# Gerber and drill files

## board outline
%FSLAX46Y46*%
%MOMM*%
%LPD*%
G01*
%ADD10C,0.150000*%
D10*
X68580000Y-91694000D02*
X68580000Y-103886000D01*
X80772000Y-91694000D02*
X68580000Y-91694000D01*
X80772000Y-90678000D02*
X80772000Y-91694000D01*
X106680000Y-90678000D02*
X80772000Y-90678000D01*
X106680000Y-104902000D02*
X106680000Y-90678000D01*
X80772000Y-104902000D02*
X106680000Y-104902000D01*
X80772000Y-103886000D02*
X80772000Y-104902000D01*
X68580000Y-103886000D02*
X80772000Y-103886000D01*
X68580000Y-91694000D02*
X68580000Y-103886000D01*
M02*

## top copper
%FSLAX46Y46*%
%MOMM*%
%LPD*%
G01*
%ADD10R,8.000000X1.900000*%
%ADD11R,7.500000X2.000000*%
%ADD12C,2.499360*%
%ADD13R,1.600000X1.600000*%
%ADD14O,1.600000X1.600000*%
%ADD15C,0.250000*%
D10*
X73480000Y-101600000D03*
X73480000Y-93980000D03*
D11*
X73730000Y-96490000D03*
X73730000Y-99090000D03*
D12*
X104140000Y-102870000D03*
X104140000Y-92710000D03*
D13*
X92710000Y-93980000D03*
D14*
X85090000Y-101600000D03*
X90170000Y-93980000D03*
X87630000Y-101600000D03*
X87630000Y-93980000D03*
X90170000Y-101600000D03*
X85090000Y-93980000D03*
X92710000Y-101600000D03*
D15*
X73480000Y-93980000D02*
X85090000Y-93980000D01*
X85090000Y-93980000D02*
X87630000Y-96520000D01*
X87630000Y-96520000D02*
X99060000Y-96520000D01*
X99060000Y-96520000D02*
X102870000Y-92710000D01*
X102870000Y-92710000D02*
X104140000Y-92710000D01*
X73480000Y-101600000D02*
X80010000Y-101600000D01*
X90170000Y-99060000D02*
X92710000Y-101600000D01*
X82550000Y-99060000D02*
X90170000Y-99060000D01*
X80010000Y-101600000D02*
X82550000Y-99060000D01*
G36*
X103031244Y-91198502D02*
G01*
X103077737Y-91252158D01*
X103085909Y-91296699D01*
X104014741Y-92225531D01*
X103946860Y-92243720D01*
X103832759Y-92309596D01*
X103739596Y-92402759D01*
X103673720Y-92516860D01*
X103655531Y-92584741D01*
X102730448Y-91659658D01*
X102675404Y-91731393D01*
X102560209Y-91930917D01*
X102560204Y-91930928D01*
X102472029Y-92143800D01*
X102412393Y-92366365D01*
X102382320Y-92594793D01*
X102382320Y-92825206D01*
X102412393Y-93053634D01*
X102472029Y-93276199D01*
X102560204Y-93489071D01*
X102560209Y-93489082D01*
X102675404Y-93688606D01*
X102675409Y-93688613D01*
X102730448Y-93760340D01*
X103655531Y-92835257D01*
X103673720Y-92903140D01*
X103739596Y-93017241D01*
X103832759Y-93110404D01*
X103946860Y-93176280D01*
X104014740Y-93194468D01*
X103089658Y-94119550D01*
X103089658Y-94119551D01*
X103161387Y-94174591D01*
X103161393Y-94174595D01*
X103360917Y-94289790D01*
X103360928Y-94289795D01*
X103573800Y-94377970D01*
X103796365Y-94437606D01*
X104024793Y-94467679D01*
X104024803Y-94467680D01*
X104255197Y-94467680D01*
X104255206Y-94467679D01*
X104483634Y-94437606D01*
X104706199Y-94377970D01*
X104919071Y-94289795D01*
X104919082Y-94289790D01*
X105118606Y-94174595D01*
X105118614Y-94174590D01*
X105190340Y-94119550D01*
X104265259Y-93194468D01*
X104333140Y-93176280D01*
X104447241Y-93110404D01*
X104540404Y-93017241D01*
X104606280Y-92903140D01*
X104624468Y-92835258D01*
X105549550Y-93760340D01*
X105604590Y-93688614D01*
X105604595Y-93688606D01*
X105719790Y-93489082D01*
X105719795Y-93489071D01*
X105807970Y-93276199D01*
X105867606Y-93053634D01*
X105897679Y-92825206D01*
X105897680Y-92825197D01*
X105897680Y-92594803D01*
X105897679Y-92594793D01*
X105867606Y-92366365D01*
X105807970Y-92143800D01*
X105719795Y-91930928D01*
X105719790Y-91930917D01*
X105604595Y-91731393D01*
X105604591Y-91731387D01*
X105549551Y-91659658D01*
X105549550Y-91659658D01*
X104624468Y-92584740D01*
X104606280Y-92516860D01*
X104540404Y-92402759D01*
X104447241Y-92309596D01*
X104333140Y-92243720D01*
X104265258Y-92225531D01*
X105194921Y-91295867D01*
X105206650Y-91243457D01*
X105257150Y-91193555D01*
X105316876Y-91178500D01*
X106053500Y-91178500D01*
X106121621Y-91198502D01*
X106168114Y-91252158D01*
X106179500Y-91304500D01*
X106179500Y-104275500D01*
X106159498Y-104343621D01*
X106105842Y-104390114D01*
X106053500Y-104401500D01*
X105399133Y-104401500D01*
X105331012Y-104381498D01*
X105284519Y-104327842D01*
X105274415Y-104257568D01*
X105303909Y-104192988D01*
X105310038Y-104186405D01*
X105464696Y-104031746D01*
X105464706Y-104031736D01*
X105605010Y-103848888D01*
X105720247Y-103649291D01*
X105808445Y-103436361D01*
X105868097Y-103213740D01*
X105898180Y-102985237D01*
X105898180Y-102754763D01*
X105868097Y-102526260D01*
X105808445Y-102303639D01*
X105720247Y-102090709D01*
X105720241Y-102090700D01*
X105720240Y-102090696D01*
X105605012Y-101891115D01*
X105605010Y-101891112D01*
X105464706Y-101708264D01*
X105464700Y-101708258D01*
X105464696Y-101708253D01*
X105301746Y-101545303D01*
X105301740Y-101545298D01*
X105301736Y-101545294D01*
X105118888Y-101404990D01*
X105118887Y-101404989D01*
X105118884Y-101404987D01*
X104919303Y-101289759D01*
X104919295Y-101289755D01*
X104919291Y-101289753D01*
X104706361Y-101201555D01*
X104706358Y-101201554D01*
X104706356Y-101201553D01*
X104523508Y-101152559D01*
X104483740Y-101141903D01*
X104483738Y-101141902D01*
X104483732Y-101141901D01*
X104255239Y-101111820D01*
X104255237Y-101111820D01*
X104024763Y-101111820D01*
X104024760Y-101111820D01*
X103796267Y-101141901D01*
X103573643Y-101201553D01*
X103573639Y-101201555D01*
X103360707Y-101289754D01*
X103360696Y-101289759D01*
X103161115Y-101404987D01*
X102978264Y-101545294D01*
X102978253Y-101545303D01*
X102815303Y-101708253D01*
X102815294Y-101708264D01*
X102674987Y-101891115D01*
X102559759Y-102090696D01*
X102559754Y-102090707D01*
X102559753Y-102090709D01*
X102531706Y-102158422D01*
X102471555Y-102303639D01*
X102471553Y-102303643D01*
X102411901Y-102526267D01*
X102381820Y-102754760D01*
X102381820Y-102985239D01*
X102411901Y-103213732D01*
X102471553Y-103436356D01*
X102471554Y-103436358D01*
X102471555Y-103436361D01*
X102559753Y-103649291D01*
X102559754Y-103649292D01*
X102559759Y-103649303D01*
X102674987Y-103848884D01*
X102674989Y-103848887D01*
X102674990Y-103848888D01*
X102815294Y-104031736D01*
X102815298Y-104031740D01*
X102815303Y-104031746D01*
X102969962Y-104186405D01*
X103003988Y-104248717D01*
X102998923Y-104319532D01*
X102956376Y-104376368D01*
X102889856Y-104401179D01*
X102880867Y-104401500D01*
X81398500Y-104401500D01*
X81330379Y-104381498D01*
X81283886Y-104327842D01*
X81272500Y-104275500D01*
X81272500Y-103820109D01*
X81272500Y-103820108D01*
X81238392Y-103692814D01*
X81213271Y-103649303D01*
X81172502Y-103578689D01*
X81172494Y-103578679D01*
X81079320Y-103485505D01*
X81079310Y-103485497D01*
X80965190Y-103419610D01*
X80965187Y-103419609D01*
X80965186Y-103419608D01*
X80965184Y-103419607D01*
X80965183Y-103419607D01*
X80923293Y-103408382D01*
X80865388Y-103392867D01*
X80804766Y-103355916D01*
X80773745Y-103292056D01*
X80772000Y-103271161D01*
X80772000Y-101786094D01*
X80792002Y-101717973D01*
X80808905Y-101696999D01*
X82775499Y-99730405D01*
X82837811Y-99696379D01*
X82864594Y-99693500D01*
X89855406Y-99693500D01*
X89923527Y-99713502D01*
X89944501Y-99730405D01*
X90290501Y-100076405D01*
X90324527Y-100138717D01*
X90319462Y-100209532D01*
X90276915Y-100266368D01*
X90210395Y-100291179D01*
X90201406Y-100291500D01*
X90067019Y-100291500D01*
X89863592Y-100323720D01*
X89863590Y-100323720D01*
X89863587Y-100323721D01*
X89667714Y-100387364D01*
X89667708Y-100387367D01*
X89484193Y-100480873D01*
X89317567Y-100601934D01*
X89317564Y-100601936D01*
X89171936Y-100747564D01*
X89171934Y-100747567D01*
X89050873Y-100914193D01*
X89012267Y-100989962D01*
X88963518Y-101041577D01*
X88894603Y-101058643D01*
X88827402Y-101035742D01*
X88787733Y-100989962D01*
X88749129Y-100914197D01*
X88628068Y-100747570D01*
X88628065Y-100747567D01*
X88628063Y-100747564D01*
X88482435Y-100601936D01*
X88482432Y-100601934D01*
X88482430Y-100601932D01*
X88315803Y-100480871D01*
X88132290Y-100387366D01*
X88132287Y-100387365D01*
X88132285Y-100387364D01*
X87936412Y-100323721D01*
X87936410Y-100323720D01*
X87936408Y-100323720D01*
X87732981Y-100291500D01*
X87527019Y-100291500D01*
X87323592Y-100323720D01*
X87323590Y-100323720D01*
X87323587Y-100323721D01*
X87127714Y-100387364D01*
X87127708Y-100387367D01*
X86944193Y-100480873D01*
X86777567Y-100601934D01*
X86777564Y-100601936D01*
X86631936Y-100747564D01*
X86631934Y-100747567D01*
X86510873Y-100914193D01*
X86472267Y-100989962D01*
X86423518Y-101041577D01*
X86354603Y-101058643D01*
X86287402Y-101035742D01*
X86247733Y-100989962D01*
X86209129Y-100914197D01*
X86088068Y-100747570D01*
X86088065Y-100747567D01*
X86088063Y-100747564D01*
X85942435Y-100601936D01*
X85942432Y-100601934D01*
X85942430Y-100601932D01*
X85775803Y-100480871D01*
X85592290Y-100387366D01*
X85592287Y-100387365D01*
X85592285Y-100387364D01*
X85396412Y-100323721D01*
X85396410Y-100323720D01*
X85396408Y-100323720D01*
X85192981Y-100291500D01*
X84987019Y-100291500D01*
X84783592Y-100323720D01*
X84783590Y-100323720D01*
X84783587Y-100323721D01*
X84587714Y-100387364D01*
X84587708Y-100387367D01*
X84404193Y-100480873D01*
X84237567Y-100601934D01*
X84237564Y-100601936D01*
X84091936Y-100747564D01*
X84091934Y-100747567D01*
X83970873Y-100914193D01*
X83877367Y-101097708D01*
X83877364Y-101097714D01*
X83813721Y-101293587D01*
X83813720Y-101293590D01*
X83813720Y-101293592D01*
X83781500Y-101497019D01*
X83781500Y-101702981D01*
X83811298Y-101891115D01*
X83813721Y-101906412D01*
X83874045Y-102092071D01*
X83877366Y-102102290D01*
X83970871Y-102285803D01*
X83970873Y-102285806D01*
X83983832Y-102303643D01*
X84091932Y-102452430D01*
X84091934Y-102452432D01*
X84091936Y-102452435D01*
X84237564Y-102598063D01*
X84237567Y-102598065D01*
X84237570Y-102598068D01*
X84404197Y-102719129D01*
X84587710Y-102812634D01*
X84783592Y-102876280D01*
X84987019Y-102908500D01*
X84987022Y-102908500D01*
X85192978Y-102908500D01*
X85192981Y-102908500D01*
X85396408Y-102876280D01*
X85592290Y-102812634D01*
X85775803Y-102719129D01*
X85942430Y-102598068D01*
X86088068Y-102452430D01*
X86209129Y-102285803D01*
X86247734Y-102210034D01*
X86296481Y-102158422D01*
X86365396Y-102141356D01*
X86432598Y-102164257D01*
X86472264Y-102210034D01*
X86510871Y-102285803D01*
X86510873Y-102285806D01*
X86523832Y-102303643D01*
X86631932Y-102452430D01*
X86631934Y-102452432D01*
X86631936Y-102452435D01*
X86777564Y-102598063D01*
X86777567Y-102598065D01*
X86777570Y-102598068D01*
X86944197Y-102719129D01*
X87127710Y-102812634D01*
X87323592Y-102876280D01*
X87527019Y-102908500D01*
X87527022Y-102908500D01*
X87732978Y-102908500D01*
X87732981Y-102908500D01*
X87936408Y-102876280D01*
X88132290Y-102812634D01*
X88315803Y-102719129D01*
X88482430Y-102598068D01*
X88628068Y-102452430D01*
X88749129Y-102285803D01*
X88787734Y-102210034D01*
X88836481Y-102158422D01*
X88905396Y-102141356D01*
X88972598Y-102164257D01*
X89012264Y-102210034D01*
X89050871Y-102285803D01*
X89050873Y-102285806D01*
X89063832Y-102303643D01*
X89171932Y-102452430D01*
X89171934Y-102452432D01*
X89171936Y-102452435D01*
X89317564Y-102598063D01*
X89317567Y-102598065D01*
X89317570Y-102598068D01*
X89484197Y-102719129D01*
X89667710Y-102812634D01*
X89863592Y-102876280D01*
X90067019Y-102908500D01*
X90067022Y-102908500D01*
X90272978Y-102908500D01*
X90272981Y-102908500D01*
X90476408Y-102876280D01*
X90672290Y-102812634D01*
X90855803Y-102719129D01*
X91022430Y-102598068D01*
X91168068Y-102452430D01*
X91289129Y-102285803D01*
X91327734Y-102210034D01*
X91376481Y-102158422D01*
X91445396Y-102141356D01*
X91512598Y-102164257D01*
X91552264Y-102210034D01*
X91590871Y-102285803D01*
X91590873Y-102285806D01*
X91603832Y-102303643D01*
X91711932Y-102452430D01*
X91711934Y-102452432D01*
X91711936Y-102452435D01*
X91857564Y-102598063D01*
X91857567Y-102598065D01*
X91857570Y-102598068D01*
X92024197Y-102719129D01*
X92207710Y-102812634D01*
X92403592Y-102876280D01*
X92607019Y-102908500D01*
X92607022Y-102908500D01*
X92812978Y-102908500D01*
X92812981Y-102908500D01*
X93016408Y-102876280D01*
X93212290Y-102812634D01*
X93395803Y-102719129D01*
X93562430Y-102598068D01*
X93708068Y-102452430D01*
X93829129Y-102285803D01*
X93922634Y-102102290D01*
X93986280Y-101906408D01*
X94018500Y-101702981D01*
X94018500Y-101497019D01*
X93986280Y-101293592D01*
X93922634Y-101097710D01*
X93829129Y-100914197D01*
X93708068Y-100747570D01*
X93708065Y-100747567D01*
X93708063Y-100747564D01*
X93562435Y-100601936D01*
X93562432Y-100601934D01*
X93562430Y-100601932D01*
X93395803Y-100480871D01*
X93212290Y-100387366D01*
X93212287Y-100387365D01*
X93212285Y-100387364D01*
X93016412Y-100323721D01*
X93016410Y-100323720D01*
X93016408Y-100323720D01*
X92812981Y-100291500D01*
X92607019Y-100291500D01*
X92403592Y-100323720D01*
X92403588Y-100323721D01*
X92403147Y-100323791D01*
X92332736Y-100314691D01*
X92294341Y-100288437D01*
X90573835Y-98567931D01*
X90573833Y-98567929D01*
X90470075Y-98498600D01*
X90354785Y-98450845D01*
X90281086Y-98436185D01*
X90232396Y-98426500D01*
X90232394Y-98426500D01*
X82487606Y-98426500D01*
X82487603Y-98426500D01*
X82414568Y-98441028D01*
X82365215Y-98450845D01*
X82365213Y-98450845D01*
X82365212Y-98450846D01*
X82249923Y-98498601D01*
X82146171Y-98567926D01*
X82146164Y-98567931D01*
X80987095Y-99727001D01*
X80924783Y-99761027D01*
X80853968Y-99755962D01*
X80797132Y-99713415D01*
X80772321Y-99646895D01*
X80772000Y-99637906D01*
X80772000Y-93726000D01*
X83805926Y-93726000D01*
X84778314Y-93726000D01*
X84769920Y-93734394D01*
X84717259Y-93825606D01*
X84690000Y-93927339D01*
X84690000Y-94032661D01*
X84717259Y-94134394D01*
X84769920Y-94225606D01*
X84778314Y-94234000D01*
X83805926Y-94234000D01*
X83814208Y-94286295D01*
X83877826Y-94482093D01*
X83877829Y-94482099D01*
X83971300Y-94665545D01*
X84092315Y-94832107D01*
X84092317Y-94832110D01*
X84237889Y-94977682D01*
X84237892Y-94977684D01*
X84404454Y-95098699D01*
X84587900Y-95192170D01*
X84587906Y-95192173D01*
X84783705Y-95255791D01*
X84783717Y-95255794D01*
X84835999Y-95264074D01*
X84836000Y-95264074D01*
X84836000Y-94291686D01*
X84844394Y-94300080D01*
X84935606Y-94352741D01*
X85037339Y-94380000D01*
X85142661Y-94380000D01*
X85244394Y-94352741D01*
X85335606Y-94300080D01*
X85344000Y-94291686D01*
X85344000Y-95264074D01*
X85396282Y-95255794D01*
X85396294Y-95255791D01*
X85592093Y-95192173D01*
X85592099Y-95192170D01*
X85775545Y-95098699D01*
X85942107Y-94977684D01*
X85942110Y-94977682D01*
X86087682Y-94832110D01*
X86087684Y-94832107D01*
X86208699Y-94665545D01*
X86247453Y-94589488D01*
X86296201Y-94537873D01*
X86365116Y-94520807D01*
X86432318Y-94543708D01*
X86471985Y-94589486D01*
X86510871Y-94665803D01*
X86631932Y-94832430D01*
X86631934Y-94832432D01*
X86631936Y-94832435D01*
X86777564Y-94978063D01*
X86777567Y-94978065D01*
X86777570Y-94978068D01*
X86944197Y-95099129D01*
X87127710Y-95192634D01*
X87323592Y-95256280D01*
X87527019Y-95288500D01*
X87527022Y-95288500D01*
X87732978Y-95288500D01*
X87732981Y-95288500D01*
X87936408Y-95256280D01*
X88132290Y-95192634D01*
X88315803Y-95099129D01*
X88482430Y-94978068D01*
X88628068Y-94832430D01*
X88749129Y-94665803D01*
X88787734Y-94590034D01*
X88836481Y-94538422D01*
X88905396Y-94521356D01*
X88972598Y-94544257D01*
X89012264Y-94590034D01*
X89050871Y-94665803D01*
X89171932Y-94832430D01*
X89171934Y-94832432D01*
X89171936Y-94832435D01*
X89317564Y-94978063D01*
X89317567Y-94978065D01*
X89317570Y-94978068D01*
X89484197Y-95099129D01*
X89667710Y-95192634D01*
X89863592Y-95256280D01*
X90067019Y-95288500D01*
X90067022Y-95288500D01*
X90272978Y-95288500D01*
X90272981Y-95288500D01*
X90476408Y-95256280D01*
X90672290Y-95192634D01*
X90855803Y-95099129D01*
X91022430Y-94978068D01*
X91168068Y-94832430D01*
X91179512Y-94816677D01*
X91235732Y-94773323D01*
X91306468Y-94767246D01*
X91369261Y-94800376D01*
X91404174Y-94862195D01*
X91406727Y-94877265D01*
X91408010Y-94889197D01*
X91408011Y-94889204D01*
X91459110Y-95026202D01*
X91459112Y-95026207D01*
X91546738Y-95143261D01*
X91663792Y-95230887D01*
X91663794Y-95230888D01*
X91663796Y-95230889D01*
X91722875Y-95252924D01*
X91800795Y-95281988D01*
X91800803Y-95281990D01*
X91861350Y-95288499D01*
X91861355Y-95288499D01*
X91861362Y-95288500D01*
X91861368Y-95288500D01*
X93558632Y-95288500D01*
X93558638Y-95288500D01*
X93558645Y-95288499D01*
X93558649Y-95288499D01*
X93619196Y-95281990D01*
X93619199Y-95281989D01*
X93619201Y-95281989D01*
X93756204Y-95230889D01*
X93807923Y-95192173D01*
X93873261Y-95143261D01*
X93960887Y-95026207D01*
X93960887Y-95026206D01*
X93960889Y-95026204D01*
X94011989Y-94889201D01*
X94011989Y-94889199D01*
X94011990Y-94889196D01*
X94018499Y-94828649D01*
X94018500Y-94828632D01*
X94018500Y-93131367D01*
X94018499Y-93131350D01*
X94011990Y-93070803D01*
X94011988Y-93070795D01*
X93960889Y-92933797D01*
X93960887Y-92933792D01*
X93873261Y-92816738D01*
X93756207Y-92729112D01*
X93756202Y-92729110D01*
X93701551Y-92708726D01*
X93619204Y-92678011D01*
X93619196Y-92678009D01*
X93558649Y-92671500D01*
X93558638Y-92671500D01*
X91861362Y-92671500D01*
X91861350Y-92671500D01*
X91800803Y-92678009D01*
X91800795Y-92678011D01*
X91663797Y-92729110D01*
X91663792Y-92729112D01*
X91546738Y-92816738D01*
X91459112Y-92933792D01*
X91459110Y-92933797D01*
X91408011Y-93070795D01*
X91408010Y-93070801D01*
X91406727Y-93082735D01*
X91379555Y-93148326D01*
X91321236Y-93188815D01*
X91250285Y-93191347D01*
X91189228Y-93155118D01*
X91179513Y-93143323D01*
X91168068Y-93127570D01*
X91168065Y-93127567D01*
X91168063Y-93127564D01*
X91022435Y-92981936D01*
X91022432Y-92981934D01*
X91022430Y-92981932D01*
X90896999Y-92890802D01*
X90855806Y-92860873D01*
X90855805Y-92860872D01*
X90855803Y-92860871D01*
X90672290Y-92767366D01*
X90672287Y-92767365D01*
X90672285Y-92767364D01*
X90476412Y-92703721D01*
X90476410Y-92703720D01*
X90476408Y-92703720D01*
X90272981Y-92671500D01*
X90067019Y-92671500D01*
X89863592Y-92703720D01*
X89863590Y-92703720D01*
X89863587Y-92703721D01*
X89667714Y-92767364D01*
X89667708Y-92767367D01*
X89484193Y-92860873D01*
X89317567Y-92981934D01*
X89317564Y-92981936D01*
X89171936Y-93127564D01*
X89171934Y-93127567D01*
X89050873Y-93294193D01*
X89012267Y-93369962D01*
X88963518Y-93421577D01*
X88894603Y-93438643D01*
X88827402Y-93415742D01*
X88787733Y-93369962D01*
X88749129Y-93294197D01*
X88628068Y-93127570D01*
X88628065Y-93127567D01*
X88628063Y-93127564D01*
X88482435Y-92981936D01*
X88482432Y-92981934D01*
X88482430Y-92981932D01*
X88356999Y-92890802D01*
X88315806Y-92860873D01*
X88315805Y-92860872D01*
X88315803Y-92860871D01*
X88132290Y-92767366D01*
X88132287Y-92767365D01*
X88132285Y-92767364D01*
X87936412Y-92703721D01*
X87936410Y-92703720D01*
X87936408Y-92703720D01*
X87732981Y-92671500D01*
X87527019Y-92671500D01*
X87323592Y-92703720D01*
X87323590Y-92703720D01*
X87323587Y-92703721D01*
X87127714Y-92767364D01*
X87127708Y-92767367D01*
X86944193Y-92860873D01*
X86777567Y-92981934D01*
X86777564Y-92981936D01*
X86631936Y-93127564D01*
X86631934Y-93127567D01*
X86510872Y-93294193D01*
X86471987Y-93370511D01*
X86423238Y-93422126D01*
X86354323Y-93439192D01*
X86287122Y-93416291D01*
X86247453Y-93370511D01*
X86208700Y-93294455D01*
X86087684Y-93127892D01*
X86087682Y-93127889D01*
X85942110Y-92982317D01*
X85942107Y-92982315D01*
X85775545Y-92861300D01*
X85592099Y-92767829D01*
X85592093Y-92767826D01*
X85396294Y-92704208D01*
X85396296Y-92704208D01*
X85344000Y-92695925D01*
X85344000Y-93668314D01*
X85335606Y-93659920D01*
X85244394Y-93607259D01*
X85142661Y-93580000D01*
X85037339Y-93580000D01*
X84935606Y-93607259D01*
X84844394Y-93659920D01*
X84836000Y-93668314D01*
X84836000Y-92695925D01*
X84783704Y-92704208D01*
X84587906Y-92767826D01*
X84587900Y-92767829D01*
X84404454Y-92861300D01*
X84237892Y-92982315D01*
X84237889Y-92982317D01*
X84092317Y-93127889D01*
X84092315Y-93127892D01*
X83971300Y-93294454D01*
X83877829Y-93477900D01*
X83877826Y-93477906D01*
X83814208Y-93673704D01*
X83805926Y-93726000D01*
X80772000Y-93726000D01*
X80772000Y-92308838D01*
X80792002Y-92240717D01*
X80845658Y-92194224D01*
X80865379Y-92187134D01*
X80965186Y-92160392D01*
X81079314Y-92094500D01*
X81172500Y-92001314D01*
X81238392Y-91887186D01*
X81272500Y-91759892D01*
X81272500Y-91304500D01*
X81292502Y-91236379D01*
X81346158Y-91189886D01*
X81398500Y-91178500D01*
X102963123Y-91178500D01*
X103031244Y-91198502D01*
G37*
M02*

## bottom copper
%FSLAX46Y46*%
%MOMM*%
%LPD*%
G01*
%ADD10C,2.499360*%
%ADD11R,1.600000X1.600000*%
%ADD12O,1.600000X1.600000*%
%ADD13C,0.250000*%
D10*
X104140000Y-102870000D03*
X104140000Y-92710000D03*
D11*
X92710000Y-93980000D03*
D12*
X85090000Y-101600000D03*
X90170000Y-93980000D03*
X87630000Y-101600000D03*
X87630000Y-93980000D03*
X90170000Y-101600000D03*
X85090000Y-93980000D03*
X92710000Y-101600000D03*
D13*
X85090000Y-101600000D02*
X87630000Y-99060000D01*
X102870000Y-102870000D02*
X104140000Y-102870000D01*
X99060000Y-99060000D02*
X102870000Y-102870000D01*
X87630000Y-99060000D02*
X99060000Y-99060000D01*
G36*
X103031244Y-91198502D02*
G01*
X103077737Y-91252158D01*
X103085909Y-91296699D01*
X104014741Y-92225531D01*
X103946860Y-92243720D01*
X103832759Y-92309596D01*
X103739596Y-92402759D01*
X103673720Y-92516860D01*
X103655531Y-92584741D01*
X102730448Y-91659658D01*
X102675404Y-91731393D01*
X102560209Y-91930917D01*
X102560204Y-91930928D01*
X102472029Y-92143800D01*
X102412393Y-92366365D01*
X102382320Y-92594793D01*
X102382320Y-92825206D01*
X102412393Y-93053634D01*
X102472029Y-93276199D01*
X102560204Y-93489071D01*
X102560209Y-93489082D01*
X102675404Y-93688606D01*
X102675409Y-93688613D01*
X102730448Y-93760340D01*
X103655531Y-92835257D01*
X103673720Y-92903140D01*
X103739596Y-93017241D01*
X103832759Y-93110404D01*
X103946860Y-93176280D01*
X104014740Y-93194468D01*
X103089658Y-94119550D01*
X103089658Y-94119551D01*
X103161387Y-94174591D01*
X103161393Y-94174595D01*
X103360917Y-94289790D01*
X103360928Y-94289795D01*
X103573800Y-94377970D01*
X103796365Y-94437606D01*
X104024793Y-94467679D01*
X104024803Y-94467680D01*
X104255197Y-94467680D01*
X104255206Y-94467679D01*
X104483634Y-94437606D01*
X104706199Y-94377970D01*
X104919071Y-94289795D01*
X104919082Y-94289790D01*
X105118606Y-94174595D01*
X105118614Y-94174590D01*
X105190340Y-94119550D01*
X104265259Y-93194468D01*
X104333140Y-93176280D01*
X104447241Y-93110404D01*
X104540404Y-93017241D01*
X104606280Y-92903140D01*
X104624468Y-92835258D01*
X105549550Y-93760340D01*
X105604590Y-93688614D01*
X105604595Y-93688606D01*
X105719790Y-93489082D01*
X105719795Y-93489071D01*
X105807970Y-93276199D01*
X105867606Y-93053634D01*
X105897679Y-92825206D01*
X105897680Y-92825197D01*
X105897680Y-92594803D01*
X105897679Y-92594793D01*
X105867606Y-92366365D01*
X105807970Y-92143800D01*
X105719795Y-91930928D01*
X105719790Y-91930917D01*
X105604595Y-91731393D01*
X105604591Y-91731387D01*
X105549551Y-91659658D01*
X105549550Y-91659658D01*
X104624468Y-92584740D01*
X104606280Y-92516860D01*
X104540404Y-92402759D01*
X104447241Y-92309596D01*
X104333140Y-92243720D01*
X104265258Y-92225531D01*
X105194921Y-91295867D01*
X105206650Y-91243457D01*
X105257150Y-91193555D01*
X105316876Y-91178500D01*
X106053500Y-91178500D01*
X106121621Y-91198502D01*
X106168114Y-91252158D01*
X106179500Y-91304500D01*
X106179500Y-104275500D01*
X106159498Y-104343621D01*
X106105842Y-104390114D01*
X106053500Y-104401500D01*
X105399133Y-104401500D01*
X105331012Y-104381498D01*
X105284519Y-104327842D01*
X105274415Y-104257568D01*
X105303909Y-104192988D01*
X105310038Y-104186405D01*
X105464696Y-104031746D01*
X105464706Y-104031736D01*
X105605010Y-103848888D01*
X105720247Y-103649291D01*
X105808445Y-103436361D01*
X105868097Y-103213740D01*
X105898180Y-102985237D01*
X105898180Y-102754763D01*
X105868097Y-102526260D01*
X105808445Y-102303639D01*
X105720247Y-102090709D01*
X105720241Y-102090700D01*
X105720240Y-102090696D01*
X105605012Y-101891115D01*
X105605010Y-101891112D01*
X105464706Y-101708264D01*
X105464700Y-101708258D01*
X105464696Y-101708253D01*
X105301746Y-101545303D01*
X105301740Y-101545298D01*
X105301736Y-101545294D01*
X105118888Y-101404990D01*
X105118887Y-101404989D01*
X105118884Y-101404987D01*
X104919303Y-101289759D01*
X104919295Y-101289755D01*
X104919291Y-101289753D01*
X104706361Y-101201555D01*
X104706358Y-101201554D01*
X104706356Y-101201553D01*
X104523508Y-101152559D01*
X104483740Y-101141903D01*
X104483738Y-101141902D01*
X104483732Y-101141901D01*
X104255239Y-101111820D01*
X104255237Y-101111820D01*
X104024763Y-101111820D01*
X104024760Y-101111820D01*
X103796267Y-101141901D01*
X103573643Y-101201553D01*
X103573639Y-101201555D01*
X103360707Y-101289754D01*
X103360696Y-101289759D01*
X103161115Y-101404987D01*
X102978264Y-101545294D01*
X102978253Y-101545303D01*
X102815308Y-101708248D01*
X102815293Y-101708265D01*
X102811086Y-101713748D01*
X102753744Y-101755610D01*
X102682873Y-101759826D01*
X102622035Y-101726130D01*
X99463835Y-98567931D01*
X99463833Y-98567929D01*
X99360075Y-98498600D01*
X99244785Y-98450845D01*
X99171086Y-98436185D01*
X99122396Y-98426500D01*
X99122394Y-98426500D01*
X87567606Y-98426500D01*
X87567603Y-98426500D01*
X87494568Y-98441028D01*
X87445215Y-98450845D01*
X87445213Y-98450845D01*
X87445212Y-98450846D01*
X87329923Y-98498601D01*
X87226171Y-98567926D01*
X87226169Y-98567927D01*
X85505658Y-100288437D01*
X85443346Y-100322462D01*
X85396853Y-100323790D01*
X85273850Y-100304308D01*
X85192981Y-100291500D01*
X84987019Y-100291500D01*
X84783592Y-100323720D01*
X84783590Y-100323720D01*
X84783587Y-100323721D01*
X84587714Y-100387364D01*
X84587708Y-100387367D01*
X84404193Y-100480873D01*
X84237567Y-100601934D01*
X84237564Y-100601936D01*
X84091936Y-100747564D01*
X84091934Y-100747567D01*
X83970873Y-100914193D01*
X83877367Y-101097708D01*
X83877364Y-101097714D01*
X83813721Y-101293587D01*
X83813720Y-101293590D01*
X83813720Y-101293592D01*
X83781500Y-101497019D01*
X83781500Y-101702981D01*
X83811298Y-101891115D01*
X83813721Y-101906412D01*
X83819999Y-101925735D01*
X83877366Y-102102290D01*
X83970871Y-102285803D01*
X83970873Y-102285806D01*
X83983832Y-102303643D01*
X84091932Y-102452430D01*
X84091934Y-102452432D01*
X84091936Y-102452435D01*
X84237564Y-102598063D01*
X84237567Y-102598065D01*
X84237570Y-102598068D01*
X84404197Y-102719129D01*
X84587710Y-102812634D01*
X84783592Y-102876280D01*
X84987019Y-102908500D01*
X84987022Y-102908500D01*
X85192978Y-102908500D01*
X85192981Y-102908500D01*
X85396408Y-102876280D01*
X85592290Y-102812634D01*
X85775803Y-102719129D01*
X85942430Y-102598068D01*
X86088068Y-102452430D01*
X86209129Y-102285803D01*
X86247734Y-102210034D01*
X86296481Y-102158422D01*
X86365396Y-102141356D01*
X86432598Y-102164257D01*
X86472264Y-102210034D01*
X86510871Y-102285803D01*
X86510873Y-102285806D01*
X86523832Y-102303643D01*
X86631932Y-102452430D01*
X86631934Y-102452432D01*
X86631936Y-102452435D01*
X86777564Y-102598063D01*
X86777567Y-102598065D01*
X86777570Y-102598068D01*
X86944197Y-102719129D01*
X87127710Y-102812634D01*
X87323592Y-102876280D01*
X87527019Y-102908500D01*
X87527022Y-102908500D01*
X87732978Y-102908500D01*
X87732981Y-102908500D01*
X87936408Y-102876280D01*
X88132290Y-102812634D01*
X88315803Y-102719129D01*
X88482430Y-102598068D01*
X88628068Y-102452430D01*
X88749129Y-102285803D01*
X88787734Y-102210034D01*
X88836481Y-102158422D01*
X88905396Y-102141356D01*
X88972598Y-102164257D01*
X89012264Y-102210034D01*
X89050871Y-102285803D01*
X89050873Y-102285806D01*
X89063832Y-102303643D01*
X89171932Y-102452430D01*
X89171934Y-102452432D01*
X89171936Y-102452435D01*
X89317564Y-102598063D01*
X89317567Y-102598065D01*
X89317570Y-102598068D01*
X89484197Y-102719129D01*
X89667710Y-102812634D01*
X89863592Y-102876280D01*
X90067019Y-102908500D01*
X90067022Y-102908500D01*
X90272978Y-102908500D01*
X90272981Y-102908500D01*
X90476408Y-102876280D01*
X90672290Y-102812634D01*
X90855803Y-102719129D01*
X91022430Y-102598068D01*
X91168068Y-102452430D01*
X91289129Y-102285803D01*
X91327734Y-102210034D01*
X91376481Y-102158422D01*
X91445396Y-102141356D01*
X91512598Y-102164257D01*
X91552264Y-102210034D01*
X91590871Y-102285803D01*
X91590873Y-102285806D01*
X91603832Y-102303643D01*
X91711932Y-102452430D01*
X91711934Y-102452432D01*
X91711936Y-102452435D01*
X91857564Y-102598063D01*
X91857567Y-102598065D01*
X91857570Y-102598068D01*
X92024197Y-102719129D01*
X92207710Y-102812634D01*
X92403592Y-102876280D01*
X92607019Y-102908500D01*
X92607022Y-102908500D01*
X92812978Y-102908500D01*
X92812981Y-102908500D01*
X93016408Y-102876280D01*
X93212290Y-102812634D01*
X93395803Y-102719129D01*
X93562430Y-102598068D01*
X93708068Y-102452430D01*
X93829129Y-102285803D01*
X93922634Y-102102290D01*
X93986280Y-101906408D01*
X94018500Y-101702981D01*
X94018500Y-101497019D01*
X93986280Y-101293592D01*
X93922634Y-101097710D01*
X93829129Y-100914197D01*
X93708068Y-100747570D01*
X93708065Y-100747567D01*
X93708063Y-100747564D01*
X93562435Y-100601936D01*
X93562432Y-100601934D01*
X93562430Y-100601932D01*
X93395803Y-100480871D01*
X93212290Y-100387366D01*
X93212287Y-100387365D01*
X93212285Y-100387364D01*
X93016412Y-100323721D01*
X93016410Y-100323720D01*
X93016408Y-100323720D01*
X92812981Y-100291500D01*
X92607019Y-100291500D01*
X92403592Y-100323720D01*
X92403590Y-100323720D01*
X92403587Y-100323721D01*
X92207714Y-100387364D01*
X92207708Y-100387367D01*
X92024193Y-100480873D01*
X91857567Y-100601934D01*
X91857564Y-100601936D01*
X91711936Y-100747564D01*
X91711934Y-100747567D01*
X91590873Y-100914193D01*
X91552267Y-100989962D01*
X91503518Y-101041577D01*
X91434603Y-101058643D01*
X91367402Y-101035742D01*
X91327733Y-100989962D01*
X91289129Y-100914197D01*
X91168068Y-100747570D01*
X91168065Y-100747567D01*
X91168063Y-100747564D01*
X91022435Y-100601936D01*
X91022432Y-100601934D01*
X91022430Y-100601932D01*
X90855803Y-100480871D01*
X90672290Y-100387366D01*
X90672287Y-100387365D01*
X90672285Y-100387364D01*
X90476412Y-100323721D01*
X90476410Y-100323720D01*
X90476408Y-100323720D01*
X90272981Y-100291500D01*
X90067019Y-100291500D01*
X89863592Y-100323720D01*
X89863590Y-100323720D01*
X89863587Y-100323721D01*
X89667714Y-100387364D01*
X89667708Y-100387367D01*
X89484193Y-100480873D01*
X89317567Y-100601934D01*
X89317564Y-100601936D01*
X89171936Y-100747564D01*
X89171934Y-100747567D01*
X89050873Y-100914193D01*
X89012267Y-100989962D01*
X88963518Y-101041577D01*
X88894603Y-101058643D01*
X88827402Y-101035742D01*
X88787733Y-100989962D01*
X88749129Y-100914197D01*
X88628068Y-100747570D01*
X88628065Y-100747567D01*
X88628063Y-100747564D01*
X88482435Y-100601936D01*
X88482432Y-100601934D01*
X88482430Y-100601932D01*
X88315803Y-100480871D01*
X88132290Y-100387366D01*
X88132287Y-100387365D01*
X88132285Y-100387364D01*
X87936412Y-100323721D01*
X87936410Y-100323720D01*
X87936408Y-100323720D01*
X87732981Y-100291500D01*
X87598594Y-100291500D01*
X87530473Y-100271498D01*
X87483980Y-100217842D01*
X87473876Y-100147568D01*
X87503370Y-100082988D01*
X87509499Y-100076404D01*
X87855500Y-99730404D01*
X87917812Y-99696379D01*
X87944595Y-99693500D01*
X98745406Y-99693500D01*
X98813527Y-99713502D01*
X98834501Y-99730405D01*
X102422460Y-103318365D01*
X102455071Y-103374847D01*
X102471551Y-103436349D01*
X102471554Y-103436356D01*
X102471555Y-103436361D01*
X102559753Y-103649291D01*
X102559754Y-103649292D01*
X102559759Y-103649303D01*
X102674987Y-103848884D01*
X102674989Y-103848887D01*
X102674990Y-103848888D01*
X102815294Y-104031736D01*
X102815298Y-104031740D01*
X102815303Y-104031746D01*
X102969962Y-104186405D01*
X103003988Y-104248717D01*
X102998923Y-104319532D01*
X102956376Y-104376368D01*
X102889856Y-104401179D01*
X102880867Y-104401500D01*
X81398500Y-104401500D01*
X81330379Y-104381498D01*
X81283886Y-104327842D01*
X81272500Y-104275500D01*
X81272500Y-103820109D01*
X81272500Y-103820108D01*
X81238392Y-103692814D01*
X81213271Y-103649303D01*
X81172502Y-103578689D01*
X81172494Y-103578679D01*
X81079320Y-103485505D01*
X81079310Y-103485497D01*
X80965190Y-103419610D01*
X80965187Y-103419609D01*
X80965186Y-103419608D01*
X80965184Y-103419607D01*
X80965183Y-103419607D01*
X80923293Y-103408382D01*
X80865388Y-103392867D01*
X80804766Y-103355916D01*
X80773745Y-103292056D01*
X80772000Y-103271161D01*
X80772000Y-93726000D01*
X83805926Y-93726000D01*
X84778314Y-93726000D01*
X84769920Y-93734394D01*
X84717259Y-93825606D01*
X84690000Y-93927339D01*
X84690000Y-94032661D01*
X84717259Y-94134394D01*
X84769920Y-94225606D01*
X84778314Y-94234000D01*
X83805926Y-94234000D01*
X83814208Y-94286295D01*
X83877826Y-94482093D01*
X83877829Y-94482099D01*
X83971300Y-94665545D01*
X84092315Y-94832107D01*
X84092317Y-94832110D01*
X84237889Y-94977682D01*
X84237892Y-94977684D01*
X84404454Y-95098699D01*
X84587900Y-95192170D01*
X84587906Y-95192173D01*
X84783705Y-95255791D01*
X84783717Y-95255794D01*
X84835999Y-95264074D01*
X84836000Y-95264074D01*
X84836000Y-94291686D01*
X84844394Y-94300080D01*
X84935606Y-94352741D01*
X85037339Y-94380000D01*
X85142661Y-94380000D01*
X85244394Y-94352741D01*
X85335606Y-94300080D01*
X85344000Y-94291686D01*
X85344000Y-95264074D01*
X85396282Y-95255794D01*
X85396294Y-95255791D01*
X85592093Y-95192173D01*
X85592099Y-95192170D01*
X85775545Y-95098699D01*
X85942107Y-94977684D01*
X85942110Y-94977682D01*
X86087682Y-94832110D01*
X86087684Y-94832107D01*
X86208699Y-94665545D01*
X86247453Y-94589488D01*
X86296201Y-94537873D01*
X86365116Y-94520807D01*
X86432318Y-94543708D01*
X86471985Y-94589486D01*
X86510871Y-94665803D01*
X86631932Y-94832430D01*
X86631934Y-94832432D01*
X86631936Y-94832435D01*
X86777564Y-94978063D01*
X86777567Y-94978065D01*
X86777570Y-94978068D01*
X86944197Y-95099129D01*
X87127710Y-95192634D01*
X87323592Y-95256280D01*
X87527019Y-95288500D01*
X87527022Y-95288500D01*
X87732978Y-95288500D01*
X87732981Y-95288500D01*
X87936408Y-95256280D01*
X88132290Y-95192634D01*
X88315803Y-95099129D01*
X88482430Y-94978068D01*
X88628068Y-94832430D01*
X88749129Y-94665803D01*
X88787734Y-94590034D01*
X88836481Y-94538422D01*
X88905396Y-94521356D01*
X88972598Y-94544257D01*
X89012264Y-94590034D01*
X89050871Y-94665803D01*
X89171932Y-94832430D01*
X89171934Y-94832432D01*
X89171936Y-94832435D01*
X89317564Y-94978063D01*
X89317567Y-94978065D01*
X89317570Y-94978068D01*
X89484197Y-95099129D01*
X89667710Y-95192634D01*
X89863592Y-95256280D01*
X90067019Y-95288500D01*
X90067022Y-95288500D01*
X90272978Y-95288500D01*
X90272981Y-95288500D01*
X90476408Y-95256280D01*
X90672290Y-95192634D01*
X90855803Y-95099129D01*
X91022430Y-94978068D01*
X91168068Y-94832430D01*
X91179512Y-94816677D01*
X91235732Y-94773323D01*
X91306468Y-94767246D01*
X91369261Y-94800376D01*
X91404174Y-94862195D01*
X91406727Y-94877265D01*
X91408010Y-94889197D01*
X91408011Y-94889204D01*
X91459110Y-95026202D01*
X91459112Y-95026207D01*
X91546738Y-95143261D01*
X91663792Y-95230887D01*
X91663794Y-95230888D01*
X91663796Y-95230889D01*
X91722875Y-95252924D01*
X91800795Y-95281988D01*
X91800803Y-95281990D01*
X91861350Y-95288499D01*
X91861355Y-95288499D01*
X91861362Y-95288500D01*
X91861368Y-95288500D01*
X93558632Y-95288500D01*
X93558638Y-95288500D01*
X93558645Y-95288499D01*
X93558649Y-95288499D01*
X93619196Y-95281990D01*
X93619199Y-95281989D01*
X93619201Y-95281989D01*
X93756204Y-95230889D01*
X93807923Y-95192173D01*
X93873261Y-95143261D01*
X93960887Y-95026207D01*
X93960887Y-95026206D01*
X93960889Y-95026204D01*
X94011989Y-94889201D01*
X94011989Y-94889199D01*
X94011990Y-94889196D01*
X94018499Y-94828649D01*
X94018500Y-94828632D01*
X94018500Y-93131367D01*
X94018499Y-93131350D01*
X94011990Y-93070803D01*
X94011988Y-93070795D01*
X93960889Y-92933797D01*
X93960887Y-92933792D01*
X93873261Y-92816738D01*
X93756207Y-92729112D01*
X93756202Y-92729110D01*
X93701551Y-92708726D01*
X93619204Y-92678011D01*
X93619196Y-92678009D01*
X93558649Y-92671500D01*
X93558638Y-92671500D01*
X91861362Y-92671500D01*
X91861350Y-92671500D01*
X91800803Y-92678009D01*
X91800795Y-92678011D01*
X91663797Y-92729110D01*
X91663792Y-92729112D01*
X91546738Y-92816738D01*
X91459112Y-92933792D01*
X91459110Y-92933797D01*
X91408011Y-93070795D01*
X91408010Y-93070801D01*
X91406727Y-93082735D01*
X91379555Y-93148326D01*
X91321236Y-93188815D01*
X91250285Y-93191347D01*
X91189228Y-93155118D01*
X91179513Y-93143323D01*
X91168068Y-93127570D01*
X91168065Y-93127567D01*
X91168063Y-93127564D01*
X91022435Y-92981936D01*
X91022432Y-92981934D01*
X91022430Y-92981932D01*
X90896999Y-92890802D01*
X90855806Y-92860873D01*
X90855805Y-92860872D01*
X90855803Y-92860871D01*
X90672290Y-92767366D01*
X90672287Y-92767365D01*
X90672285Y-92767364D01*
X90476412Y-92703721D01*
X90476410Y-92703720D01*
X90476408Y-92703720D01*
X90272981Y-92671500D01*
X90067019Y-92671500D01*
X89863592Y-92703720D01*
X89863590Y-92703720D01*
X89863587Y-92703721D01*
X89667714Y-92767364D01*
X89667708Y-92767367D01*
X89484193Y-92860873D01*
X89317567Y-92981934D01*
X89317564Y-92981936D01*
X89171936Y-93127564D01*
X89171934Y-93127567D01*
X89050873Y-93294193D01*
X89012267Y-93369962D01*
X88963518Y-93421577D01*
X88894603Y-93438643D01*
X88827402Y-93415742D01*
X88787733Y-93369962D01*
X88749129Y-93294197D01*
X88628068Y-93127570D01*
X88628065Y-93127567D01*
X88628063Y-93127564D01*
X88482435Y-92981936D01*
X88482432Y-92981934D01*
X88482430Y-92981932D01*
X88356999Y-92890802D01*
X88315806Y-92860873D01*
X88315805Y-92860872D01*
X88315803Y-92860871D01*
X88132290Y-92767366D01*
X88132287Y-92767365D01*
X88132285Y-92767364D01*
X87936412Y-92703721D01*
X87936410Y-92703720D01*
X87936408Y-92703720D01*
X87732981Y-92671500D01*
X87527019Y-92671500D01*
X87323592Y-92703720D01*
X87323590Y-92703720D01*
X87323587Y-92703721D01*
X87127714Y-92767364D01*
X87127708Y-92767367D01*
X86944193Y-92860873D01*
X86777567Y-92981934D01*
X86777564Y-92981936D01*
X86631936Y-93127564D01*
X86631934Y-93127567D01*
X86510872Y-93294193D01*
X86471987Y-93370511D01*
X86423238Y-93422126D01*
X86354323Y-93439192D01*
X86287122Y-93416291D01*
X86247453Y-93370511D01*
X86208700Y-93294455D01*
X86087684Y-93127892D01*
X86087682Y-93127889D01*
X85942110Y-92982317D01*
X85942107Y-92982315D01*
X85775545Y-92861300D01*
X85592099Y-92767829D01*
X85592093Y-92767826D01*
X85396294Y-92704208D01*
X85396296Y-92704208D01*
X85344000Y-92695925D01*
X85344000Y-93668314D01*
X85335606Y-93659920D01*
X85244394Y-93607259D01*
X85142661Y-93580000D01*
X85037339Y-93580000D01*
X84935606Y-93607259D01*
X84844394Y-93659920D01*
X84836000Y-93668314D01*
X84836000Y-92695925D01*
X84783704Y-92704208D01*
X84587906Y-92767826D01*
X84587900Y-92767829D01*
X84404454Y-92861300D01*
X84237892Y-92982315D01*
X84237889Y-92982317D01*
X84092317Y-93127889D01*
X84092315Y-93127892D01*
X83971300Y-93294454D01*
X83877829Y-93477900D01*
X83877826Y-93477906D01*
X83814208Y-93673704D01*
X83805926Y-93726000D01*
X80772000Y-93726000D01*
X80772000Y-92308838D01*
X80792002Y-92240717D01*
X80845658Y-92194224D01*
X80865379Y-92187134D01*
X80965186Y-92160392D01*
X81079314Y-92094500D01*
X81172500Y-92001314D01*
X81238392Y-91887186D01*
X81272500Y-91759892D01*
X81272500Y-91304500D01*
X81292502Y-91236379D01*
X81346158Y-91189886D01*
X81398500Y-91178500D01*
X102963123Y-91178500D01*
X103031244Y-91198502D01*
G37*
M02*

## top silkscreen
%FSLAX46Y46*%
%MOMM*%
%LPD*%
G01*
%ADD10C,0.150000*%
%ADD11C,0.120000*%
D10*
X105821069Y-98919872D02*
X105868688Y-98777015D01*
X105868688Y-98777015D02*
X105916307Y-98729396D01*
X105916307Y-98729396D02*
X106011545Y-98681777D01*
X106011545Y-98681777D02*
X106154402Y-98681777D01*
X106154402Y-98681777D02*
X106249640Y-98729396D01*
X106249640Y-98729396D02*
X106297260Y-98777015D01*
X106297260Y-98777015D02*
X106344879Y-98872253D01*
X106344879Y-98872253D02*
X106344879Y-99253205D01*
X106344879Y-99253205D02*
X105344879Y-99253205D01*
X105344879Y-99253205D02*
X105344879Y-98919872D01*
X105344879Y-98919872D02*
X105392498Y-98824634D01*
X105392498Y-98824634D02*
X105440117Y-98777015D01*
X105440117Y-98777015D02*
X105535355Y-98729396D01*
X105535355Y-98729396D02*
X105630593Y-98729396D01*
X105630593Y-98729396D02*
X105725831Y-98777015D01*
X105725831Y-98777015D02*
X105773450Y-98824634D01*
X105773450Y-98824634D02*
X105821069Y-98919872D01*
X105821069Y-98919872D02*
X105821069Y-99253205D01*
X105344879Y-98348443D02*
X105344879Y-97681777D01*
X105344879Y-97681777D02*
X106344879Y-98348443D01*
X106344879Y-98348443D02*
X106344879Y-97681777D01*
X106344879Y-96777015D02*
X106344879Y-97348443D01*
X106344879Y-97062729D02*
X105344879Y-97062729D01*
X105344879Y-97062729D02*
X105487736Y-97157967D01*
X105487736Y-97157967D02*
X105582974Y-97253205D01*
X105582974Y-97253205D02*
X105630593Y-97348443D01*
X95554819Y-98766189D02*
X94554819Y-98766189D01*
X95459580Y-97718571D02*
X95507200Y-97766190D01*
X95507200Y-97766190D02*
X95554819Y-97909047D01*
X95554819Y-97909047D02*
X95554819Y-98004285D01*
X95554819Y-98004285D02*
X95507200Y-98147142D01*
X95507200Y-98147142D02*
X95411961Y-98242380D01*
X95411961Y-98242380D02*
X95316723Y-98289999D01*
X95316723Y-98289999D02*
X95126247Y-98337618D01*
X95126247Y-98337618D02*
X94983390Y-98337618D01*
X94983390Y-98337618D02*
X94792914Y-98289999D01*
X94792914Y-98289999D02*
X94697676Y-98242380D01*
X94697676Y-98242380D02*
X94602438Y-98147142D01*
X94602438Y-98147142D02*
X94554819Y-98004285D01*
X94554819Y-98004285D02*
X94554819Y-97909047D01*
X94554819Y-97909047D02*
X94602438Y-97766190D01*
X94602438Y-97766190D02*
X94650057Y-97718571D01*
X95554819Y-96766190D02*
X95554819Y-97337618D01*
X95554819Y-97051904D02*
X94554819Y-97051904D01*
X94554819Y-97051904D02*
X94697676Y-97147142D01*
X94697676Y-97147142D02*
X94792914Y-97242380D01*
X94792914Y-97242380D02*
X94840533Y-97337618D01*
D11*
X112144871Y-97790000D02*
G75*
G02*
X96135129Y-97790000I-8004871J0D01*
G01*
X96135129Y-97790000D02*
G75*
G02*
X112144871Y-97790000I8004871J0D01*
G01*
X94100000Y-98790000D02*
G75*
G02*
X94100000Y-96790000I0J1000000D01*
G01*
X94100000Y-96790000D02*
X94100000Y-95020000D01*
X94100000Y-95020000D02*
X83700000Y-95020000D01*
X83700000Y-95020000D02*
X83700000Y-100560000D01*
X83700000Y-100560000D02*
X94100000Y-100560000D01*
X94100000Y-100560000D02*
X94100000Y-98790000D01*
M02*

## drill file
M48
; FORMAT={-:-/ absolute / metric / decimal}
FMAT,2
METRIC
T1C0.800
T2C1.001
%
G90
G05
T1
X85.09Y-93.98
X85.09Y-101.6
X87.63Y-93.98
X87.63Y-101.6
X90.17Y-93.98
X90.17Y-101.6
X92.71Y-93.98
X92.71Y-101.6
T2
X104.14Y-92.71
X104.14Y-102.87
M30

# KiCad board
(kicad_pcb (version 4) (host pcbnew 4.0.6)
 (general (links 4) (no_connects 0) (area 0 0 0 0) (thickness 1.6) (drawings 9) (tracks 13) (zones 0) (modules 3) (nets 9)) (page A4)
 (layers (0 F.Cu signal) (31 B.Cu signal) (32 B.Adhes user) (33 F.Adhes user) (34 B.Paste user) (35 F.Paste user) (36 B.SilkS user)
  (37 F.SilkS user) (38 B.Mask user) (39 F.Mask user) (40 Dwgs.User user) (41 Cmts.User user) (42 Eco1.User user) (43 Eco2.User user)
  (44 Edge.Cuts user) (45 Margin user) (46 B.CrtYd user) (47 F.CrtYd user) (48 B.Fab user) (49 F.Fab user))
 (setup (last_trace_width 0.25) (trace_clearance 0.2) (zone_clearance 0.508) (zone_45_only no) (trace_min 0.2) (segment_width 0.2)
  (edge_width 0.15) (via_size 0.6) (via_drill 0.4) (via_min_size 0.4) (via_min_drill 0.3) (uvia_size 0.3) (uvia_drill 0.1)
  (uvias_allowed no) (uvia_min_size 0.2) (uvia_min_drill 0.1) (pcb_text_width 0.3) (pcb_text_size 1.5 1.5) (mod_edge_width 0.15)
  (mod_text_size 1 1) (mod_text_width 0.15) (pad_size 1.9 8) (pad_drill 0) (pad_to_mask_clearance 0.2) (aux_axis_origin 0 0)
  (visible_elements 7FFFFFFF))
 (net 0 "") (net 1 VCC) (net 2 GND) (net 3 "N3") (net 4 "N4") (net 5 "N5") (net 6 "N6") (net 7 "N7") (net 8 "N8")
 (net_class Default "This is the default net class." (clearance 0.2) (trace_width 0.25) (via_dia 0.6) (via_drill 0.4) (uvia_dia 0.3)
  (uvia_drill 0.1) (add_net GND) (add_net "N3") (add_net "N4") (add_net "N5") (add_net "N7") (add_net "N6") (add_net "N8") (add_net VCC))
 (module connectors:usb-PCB (layer F.Cu) (at 68.58 91.44 270)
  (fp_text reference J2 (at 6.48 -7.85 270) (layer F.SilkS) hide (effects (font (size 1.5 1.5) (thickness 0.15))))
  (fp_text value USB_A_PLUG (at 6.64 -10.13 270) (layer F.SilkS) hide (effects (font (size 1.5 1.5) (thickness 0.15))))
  (pad 1 connect rect (at 10.16 -4.9 270) (size 1.9 8) (layers F.Cu F.Mask) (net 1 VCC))
  (pad 4 connect rect (at 2.54 -4.9 270) (size 1.9 8) (layers F.Cu F.Mask) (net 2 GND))
  (pad 3 connect rect (at 5.05 -5.15 270) (size 2 7.5) (layers F.Cu F.Mask))
  (pad 2 connect rect (at 7.65 -5.15 270) (size 2 7.5) (layers F.Cu F.Mask)))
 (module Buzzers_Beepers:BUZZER (layer F.Cu) (at 104.14 97.79 270)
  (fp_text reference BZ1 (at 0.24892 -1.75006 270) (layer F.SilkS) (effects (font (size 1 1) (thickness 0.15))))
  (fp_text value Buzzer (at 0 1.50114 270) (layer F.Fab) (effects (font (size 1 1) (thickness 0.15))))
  (fp_circle (center 0 0) (end 8.001 0.24892) (layer F.SilkS) (width 0.12))
  (pad 2 thru_hole circle (at 5.08 0 270) (size 2.49936 2.49936) (drill 1.00076) (layers *.Cu *.Mask) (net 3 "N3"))
  (pad 1 thru_hole circle (at -5.08 0 270) (size 2.49936 2.49936) (drill 1.00076) (layers *.Cu *.Mask) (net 2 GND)))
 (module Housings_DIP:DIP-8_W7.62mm (layer F.Cu) (at 92.71 93.98 270)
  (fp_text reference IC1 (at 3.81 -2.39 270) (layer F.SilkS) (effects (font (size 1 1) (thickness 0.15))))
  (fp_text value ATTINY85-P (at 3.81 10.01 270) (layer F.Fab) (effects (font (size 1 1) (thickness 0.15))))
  (fp_arc (start 3.81 -1.39) (end 2.81 -1.39) (angle -180) (layer F.SilkS) (width 0.12))
  (fp_line (start 2.81 -1.39) (end 1.04 -1.39) (layer F.SilkS) (width 0.12))
  (fp_line (start 1.04 -1.39) (end 1.04 9.01) (layer F.SilkS) (width 0.12))
  (fp_line (start 1.04 9.01) (end 6.58 9.01) (layer F.SilkS) (width 0.12))
  (fp_line (start 6.58 9.01) (end 6.58 -1.39) (layer F.SilkS) (width 0.12))
  (fp_line (start 6.58 -1.39) (end 4.81 -1.39) (layer F.SilkS) (width 0.12))
  (pad 1 thru_hole rect (at 0 0 270) (size 1.6 1.6) (drill 0.8) (layers *.Cu *.Mask) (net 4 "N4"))
  (pad 5 thru_hole oval (at 7.62 7.62 270) (size 1.6 1.6) (drill 0.8) (layers *.Cu *.Mask) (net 3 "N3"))
  (pad 2 thru_hole oval (at 0 2.54 270) (size 1.6 1.6) (drill 0.8) (layers *.Cu *.Mask) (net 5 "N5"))
  (pad 6 thru_hole oval (at 7.62 5.08 270) (size 1.6 1.6) (drill 0.8) (layers *.Cu *.Mask) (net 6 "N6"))
  (pad 3 thru_hole oval (at 0 5.08 270) (size 1.6 1.6) (drill 0.8) (layers *.Cu *.Mask) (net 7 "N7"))
  (pad 7 thru_hole oval (at 7.62 2.54 270) (size 1.6 1.6) (drill 0.8) (layers *.Cu *.Mask) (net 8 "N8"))
  (pad 4 thru_hole oval (at 0 7.62 270) (size 1.6 1.6) (drill 0.8) (layers *.Cu *.Mask) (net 2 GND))
  (pad 8 thru_hole oval (at 7.62 0 270) (size 1.6 1.6) (drill 0.8) (layers *.Cu *.Mask) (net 1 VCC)))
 (gr_line (start 68.58 91.694) (end 68.58 103.886) (angle 90) (layer Edge.Cuts) (width 0.15))
 (gr_line (start 80.772 91.694) (end 68.58 91.694) (angle 90) (layer Edge.Cuts) (width 0.15))
 (gr_line (start 80.772 90.678) (end 80.772 91.694) (angle 90) (layer Edge.Cuts) (width 0.15))
 (gr_line (start 106.68 90.678) (end 80.772 90.678) (angle 90) (layer Edge.Cuts) (width 0.15))
 (gr_line (start 106.68 104.902) (end 106.68 90.678) (angle 90) (layer Edge.Cuts) (width 0.15))
 (gr_line (start 80.772 104.902) (end 106.68 104.902) (angle 90) (layer Edge.Cuts) (width 0.15))
 (gr_line (start 80.772 103.886) (end 80.772 104.902) (angle 90) (layer Edge.Cuts) (width 0.15))
 (gr_line (start 68.58 103.886) (end 80.772 103.886) (angle 90) (layer Edge.Cuts) (width 0.15))
 (gr_line (start 68.58 91.694) (end 68.58 103.886) (angle 90) (layer Edge.Cuts) (width 0.15))
 (segment (start 85.09 101.6) (end 87.63 99.06) (width 0.25) (layer B.Cu) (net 3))
 (segment (start 102.87 102.87) (end 104.14 102.87) (width 0.25) (layer B.Cu) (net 3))
 (segment (start 99.06 99.06) (end 102.87 102.87) (width 0.25) (layer B.Cu) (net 3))
 (segment (start 87.63 99.06) (end 99.06 99.06) (width 0.25) (layer B.Cu) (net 3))
 (segment (start 73.48 93.98) (end 85.09 93.98) (width 0.25) (layer F.Cu) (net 2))
 (segment (start 85.09 93.98) (end 87.63 96.52) (width 0.25) (layer F.Cu) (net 2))
 (segment (start 87.63 96.52) (end 99.06 96.52) (width 0.25) (layer F.Cu) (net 2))
 (segment (start 99.06 96.52) (end 102.87 92.71) (width 0.25) (layer F.Cu) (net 2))
 (segment (start 102.87 92.71) (end 104.14 92.71) (width 0.25) (layer F.Cu) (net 2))
 (segment (start 73.48 101.6) (end 80.01 101.6) (width 0.25) (layer F.Cu) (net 1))
 (segment (start 90.17 99.06) (end 92.71 101.6) (width 0.25) (layer F.Cu) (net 1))
 (segment (start 82.55 99.06) (end 90.17 99.06) (width 0.25) (layer F.Cu) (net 1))
 (segment (start 80.01 101.6) (end 82.55 99.06) (width 0.25) (layer F.Cu) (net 1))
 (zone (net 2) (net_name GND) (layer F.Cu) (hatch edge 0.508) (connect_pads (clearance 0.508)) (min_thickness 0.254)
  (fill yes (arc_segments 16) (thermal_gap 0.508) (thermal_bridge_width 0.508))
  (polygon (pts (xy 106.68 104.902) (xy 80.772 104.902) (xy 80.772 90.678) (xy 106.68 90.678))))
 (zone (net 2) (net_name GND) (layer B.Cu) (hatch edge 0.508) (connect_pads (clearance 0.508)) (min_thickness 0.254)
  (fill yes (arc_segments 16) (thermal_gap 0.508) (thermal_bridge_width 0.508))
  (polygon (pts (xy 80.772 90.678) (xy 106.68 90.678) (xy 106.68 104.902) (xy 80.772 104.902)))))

